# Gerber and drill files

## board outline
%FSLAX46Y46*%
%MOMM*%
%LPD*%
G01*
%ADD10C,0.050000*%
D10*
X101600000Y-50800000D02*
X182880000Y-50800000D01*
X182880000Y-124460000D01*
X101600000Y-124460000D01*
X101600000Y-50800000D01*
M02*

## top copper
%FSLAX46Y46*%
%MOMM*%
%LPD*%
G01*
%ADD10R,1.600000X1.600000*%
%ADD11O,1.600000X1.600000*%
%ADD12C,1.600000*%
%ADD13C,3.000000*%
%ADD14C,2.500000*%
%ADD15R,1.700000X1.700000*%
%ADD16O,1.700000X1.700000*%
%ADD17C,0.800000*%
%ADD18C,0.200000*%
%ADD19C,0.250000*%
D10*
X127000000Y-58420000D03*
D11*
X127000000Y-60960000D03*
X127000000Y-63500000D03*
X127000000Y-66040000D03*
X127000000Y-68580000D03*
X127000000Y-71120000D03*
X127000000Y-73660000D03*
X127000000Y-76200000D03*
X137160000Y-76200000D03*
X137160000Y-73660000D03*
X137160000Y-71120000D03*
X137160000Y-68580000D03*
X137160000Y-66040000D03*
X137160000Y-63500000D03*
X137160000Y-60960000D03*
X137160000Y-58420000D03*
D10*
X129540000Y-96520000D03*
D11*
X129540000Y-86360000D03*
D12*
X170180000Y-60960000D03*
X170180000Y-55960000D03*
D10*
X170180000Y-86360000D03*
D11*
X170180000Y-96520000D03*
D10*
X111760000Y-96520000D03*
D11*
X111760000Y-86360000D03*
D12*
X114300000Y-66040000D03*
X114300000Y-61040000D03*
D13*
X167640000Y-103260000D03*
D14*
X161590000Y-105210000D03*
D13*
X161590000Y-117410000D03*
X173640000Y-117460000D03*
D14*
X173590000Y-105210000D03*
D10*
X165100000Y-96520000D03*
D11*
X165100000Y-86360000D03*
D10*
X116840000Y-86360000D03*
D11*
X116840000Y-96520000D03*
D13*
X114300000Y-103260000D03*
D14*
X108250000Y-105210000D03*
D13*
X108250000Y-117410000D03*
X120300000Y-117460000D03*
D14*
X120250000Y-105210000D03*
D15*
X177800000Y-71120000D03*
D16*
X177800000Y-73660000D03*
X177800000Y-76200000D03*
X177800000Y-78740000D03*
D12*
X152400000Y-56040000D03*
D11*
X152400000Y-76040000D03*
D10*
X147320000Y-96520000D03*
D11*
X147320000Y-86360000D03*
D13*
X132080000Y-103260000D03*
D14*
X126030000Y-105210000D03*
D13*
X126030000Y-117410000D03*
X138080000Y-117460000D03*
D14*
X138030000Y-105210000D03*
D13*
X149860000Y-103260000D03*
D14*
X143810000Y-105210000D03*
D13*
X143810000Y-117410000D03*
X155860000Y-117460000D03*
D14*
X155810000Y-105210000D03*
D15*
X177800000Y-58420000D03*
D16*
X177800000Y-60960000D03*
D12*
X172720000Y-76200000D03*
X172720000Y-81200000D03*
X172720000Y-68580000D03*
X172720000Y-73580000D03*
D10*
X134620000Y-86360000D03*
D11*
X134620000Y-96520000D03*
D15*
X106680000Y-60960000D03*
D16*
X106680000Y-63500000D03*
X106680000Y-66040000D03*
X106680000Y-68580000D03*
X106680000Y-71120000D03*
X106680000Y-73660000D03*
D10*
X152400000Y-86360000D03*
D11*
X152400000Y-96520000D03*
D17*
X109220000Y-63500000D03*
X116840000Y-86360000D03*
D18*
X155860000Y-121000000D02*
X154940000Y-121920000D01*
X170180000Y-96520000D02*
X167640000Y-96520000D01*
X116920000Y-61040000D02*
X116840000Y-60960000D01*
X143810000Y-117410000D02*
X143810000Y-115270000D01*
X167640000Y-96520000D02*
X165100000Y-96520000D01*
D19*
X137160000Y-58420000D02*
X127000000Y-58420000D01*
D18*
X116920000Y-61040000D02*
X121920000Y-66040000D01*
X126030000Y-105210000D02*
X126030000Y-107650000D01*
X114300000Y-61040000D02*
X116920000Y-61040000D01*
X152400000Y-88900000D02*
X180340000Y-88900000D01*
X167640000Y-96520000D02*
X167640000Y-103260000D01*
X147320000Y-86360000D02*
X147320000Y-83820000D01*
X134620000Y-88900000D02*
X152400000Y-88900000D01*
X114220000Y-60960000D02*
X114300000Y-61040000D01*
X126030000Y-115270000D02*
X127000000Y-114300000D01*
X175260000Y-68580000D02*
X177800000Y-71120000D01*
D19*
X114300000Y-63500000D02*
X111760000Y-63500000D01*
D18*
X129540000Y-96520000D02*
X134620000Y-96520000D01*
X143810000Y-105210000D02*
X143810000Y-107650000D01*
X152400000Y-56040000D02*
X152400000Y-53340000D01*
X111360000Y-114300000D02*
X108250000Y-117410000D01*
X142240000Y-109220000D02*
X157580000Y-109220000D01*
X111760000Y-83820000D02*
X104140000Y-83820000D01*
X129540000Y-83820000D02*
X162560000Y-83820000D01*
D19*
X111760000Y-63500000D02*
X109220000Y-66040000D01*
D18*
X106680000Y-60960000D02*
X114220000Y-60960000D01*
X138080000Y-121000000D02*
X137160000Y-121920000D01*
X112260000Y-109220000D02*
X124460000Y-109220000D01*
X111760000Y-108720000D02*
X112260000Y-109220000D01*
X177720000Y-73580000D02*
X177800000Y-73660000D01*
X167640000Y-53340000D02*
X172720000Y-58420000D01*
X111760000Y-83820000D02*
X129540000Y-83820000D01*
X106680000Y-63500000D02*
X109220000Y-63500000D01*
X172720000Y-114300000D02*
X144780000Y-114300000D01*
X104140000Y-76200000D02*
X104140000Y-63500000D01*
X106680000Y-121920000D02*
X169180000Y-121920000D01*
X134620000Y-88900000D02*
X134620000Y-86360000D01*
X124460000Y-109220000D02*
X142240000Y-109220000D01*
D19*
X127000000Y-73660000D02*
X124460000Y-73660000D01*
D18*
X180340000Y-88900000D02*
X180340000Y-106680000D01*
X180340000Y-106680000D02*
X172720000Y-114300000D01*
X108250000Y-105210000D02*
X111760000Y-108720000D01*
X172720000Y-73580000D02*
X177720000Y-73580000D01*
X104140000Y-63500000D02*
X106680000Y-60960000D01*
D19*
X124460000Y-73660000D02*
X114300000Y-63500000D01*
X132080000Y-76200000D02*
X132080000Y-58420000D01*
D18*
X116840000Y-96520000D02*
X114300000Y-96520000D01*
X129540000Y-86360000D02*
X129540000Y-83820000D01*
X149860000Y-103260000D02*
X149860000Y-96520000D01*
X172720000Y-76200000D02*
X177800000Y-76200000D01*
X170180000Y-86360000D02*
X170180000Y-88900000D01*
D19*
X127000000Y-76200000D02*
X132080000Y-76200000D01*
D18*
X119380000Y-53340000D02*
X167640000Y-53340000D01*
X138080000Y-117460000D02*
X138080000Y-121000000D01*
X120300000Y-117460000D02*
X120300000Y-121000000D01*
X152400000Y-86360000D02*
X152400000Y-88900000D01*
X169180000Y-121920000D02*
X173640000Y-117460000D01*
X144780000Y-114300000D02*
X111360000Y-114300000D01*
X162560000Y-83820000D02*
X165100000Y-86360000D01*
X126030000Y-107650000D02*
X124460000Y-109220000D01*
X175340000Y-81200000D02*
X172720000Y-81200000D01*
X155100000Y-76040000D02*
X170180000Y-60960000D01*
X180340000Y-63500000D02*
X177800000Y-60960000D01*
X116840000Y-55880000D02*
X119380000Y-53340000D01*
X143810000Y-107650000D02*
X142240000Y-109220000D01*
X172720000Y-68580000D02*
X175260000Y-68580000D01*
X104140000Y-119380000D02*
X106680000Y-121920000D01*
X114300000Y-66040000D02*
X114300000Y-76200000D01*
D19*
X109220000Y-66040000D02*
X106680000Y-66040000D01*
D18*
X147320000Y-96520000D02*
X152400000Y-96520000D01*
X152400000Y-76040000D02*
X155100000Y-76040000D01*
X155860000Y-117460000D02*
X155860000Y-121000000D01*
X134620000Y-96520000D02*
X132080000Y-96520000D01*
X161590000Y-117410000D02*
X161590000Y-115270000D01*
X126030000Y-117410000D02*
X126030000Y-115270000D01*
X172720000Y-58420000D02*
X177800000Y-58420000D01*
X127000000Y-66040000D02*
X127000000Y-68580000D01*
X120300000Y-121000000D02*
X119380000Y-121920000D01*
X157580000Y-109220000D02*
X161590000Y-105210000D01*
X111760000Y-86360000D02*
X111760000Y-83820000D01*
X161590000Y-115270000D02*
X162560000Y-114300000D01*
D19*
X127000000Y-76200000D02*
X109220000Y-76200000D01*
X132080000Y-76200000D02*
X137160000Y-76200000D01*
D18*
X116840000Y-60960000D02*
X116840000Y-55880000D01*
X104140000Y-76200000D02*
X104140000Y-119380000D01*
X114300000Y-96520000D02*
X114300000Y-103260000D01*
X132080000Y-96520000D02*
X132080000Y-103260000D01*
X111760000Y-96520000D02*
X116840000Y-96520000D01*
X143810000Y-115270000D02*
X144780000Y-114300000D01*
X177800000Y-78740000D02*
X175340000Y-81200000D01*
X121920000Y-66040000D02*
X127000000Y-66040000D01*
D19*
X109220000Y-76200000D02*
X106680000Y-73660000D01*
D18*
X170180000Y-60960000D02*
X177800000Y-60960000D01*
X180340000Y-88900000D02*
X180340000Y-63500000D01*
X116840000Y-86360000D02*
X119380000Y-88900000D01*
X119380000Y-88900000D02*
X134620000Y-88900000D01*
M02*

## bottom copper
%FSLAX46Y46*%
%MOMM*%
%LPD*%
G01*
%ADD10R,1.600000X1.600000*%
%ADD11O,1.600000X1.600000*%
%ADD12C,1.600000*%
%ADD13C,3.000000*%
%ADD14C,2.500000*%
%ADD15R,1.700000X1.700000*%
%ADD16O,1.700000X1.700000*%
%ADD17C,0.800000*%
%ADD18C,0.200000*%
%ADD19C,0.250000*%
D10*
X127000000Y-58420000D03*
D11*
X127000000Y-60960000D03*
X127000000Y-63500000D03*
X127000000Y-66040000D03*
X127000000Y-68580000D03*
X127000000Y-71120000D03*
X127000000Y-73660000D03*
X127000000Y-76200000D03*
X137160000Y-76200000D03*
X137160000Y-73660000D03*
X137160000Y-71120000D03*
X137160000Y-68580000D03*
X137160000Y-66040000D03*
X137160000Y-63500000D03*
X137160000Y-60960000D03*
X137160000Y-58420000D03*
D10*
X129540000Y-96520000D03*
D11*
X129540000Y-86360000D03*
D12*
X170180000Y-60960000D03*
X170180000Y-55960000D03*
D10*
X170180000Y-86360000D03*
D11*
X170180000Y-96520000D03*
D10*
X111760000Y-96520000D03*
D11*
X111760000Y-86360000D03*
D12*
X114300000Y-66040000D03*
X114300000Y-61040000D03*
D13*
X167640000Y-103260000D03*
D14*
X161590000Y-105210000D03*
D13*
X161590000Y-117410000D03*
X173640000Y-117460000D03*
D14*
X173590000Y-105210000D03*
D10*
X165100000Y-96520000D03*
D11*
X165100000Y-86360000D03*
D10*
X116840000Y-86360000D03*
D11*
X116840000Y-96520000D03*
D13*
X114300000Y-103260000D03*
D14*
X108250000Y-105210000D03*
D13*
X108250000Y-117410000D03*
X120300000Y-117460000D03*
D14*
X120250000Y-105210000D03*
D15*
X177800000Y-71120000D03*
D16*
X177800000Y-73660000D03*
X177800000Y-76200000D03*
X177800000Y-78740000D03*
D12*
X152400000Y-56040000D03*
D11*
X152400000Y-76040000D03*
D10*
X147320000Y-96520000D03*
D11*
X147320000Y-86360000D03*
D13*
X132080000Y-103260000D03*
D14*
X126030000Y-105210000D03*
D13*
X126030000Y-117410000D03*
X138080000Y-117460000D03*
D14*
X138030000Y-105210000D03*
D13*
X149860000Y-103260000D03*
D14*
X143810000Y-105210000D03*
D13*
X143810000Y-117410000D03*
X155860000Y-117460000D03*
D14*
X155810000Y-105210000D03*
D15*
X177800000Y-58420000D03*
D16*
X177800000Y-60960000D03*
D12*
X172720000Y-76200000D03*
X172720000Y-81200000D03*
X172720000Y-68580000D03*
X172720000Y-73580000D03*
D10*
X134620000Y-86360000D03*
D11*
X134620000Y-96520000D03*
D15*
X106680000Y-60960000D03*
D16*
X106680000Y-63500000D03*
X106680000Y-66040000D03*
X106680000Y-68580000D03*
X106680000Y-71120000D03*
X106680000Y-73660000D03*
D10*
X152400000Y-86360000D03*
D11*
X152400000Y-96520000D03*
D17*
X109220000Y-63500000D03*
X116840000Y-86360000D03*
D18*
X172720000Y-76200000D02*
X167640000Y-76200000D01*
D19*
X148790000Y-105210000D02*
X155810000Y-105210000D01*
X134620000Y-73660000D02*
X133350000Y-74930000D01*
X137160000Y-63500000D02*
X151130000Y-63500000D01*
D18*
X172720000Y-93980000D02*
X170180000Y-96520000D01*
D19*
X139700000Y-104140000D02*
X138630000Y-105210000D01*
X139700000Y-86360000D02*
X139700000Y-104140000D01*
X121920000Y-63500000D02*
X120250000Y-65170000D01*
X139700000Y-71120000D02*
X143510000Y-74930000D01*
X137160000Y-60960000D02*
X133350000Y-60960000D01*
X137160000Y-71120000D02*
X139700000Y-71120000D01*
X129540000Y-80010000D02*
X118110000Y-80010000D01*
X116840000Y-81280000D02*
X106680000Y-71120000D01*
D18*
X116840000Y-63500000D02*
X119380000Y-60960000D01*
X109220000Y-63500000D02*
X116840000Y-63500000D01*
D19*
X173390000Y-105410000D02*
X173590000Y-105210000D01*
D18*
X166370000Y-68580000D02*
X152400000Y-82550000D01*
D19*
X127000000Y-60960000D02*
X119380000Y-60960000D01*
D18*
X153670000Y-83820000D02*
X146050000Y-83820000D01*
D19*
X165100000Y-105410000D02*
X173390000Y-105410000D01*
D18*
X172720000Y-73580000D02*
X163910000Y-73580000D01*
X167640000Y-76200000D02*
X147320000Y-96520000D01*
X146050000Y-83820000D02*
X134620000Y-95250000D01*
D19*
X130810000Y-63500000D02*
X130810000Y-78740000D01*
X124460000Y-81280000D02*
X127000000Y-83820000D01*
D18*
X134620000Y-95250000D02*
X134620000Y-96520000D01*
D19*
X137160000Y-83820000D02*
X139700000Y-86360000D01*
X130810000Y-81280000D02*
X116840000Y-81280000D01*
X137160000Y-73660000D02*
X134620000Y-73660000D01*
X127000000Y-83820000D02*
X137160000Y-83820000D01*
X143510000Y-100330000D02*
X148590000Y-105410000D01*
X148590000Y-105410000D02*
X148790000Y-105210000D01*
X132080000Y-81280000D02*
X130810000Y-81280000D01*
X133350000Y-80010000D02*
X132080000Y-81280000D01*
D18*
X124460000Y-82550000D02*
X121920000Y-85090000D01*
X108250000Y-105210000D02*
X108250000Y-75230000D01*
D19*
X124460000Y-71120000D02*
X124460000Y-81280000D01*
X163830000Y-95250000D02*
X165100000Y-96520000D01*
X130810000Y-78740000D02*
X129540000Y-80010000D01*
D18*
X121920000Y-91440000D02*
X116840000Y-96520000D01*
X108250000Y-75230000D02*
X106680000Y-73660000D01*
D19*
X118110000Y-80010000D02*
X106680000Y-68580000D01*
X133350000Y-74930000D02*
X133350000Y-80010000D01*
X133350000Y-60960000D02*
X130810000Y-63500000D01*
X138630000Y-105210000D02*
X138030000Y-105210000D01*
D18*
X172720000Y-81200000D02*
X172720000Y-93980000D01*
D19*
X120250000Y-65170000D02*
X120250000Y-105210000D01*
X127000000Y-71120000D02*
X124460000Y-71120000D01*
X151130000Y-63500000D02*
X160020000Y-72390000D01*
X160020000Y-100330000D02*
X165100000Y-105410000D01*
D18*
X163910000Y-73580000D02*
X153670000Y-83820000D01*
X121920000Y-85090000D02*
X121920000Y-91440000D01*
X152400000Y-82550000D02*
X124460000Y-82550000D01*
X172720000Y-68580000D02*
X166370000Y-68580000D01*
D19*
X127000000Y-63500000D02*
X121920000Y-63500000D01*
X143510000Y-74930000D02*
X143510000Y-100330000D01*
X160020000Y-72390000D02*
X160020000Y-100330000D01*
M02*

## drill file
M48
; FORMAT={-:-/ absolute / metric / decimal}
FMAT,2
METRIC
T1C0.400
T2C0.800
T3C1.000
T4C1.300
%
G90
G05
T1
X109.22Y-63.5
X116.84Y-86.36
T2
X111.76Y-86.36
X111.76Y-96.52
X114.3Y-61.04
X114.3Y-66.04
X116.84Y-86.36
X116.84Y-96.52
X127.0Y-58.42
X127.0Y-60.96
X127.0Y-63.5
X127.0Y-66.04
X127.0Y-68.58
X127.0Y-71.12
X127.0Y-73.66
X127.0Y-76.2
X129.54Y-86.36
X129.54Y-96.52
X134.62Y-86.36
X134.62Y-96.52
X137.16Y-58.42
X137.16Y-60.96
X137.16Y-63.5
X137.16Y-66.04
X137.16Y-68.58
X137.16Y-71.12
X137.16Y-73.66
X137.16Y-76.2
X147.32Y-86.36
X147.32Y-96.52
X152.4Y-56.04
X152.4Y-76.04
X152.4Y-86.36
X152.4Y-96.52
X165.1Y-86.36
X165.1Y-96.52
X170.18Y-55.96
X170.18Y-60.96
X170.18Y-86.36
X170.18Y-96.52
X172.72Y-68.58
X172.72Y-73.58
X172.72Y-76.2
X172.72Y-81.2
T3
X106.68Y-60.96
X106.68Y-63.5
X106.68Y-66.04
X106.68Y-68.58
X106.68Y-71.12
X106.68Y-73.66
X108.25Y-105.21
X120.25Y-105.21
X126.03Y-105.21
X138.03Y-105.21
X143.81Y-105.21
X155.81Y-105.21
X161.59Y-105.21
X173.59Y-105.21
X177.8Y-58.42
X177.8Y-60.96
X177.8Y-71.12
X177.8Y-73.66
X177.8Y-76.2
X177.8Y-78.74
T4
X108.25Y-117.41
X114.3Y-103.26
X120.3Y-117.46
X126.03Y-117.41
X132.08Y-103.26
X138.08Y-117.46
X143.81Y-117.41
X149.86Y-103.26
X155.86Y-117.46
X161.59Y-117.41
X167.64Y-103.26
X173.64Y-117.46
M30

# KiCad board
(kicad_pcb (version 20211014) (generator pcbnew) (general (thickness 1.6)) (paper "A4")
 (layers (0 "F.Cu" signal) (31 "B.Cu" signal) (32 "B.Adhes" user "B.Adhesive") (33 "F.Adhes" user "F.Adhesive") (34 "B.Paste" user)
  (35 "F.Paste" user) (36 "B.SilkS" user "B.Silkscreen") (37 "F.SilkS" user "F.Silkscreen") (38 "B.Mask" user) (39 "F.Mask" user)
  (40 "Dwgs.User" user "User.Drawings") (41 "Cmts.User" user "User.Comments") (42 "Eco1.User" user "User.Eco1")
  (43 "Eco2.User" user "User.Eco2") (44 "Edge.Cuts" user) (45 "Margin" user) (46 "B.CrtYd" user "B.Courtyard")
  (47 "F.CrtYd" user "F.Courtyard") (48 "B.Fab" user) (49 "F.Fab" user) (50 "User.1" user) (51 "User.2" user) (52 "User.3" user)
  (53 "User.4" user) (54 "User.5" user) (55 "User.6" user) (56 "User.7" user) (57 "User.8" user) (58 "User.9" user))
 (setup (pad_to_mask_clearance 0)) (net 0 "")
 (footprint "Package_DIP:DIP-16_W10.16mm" (layer "F.Cu") (at 127 58.42)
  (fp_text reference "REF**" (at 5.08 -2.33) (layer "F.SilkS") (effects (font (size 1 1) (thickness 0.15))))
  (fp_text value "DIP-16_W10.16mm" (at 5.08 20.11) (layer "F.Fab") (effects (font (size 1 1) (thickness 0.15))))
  (pad "1" thru_hole rect (at 0 0) (size 1.6 1.6) (drill 0.8) (layers *.Cu *.Mask))
  (pad "2" thru_hole oval (at 0 2.54) (size 1.6 1.6) (drill 0.8) (layers *.Cu *.Mask))
  (pad "3" thru_hole oval (at 0 5.08) (size 1.6 1.6) (drill 0.8) (layers *.Cu *.Mask))
  (pad "4" thru_hole oval (at 0 7.62) (size 1.6 1.6) (drill 0.8) (layers *.Cu *.Mask))
  (pad "5" thru_hole oval (at 0 10.16) (size 1.6 1.6) (drill 0.8) (layers *.Cu *.Mask))
  (pad "6" thru_hole oval (at 0 12.7) (size 1.6 1.6) (drill 0.8) (layers *.Cu *.Mask))
  (pad "7" thru_hole oval (at 0 15.24) (size 1.6 1.6) (drill 0.8) (layers *.Cu *.Mask))
  (pad "8" thru_hole oval (at 0 17.78) (size 1.6 1.6) (drill 0.8) (layers *.Cu *.Mask))
  (pad "9" thru_hole oval (at 10.16 17.78) (size 1.6 1.6) (drill 0.8) (layers *.Cu *.Mask))
  (pad "10" thru_hole oval (at 10.16 15.24) (size 1.6 1.6) (drill 0.8) (layers *.Cu *.Mask))
  (pad "11" thru_hole oval (at 10.16 12.7) (size 1.6 1.6) (drill 0.8) (layers *.Cu *.Mask))
  (pad "12" thru_hole oval (at 10.16 10.16) (size 1.6 1.6) (drill 0.8) (layers *.Cu *.Mask))
  (pad "13" thru_hole oval (at 10.16 7.62) (size 1.6 1.6) (drill 0.8) (layers *.Cu *.Mask))
  (pad "14" thru_hole oval (at 10.16 5.08) (size 1.6 1.6) (drill 0.8) (layers *.Cu *.Mask))
  (pad "15" thru_hole oval (at 10.16 2.54) (size 1.6 1.6) (drill 0.8) (layers *.Cu *.Mask))
  (pad "16" thru_hole oval (at 10.16 0) (size 1.6 1.6) (drill 0.8) (layers *.Cu *.Mask)))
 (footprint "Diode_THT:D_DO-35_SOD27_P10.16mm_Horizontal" (layer "F.Cu") (at 129.54 96.52 90)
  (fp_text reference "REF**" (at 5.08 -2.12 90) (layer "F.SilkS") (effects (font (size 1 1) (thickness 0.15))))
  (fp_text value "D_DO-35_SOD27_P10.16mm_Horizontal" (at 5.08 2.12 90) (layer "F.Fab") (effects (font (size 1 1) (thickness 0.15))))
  (pad "1" thru_hole rect (at 0 0 90) (size 1.6 1.6) (drill 0.8) (layers *.Cu *.Mask))
  (pad "2" thru_hole oval (at 10.16 0 90) (size 1.6 1.6) (drill 0.8) (layers *.Cu *.Mask)))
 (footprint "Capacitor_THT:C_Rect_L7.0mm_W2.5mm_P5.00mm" (layer "F.Cu") (at 170.18 60.96 90)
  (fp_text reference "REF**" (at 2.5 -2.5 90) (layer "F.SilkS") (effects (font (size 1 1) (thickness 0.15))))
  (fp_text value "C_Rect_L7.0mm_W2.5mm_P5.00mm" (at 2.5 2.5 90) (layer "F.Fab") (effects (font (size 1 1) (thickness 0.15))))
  (pad "1" thru_hole circle (at 0 0 90) (size 1.6 1.6) (drill 0.8) (layers *.Cu *.Mask))
  (pad "2" thru_hole circle (at 5 0 90) (size 1.6 1.6) (drill 0.8) (layers *.Cu *.Mask)))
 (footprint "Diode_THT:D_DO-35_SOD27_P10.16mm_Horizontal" (layer "F.Cu") (at 170.18 86.36 -90)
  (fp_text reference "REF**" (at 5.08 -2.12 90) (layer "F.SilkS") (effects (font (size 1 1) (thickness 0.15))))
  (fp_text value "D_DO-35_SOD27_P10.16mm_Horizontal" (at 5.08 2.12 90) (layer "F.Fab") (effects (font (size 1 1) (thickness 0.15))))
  (pad "1" thru_hole rect (at 0 0 270) (size 1.6 1.6) (drill 0.8) (layers *.Cu *.Mask))
  (pad "2" thru_hole oval (at 10.16 0 270) (size 1.6 1.6) (drill 0.8) (layers *.Cu *.Mask)))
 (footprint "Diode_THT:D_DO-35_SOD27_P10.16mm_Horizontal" (layer "F.Cu") (at 111.76 96.52 90)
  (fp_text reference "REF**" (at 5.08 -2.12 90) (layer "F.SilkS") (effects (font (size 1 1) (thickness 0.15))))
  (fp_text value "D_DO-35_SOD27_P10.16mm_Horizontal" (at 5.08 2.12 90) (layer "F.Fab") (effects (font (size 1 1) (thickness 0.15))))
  (pad "1" thru_hole rect (at 0 0 90) (size 1.6 1.6) (drill 0.8) (layers *.Cu *.Mask))
  (pad "2" thru_hole oval (at 10.16 0 90) (size 1.6 1.6) (drill 0.8) (layers *.Cu *.Mask)))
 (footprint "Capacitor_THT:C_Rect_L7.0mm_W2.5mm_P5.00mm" (layer "F.Cu") (at 114.3 66.04 90)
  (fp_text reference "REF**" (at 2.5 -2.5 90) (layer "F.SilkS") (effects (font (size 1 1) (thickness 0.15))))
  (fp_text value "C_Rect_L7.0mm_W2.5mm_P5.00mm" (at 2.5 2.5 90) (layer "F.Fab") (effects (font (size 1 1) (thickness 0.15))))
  (pad "1" thru_hole circle (at 0 0 90) (size 1.6 1.6) (drill 0.8) (layers *.Cu *.Mask))
  (pad "2" thru_hole circle (at 5 0 90) (size 1.6 1.6) (drill 0.8) (layers *.Cu *.Mask)))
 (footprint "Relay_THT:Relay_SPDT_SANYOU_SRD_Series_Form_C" (layer "F.Cu") (at 167.64 103.26 -90)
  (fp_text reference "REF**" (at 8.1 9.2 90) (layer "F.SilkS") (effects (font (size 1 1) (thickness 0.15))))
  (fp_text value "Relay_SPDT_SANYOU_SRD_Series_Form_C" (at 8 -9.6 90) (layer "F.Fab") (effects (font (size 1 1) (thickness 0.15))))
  (pad "1" thru_hole circle (at 0 0) (size 3 3) (drill 1.3) (layers *.Cu *.Mask))
  (pad "2" thru_hole circle (at 1.95 6.05) (size 2.5 2.5) (drill 1) (layers *.Cu *.Mask))
  (pad "3" thru_hole circle (at 14.15 6.05) (size 3 3) (drill 1.3) (layers *.Cu *.Mask))
  (pad "4" thru_hole circle (at 14.2 -6) (size 3 3) (drill 1.3) (layers *.Cu *.Mask))
  (pad "5" thru_hole circle (at 1.95 -5.95) (size 2.5 2.5) (drill 1) (layers *.Cu *.Mask)))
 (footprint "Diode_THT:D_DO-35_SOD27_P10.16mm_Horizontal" (layer "F.Cu") (at 165.1 96.52 90)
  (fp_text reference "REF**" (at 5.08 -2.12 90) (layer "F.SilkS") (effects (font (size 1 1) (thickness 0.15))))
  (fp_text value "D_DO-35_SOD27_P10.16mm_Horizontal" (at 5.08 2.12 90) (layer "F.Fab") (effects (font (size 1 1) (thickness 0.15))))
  (pad "1" thru_hole rect (at 0 0 90) (size 1.6 1.6) (drill 0.8) (layers *.Cu *.Mask))
  (pad "2" thru_hole oval (at 10.16 0 90) (size 1.6 1.6) (drill 0.8) (layers *.Cu *.Mask)))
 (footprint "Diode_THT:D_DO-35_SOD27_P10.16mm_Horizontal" (layer "F.Cu") (at 116.84 86.36 -90)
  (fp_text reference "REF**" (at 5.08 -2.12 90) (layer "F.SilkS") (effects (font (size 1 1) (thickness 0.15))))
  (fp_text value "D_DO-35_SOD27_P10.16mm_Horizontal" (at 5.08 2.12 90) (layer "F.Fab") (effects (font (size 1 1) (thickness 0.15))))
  (pad "1" thru_hole rect (at 0 0 270) (size 1.6 1.6) (drill 0.8) (layers *.Cu *.Mask))
  (pad "2" thru_hole oval (at 10.16 0 270) (size 1.6 1.6) (drill 0.8) (layers *.Cu *.Mask)))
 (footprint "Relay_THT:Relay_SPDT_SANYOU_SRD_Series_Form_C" (layer "F.Cu") (at 114.3 103.26 -90)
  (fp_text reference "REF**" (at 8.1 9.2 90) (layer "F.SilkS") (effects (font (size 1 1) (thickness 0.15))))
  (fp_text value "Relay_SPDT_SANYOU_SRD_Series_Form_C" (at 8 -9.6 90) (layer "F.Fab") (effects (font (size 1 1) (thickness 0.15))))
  (pad "1" thru_hole circle (at 0 0) (size 3 3) (drill 1.3) (layers *.Cu *.Mask))
  (pad "2" thru_hole circle (at 1.95 6.05) (size 2.5 2.5) (drill 1) (layers *.Cu *.Mask))
  (pad "3" thru_hole circle (at 14.15 6.05) (size 3 3) (drill 1.3) (layers *.Cu *.Mask))
  (pad "4" thru_hole circle (at 14.2 -6) (size 3 3) (drill 1.3) (layers *.Cu *.Mask))
  (pad "5" thru_hole circle (at 1.95 -5.95) (size 2.5 2.5) (drill 1) (layers *.Cu *.Mask)))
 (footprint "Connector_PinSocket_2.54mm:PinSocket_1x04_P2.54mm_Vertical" (layer "F.Cu") (at 177.8 71.12)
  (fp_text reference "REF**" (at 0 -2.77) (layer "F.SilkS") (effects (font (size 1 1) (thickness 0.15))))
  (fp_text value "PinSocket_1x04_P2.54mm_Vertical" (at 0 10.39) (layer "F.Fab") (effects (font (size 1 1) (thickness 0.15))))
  (pad "1" thru_hole rect (at 0 0) (size 1.7 1.7) (drill 1) (layers *.Cu *.Mask))
  (pad "2" thru_hole oval (at 0 2.54) (size 1.7 1.7) (drill 1) (layers *.Cu *.Mask))
  (pad "3" thru_hole oval (at 0 5.08) (size 1.7 1.7) (drill 1) (layers *.Cu *.Mask))
  (pad "4" thru_hole oval (at 0 7.62) (size 1.7 1.7) (drill 1) (layers *.Cu *.Mask)))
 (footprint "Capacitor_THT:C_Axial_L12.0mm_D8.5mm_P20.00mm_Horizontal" (layer "F.Cu") (at 152.4 56.04 -90)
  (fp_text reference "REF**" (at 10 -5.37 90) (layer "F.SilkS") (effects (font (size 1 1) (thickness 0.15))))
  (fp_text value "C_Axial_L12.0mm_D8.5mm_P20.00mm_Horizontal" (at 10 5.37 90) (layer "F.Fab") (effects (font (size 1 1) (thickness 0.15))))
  (pad "1" thru_hole circle (at 0 0 270) (size 1.6 1.6) (drill 0.8) (layers *.Cu *.Mask))
  (pad "2" thru_hole oval (at 20 0 270) (size 1.6 1.6) (drill 0.8) (layers *.Cu *.Mask)))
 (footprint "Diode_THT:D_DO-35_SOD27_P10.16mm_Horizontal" (layer "F.Cu") (at 147.32 96.52 90)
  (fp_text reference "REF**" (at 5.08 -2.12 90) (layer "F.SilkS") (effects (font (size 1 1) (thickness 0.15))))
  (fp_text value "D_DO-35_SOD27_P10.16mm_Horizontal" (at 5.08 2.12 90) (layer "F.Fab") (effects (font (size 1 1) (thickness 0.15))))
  (pad "1" thru_hole rect (at 0 0 90) (size 1.6 1.6) (drill 0.8) (layers *.Cu *.Mask))
  (pad "2" thru_hole oval (at 10.16 0 90) (size 1.6 1.6) (drill 0.8) (layers *.Cu *.Mask)))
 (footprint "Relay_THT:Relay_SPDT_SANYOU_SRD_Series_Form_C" (layer "F.Cu") (at 132.08 103.26 -90)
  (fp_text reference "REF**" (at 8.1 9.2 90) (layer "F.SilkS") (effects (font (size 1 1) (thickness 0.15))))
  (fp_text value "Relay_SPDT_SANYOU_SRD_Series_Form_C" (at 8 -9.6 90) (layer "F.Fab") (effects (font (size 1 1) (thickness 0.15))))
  (pad "1" thru_hole circle (at 0 0) (size 3 3) (drill 1.3) (layers *.Cu *.Mask))
  (pad "2" thru_hole circle (at 1.95 6.05) (size 2.5 2.5) (drill 1) (layers *.Cu *.Mask))
  (pad "3" thru_hole circle (at 14.15 6.05) (size 3 3) (drill 1.3) (layers *.Cu *.Mask))
  (pad "4" thru_hole circle (at 14.2 -6) (size 3 3) (drill 1.3) (layers *.Cu *.Mask))
  (pad "5" thru_hole circle (at 1.95 -5.95) (size 2.5 2.5) (drill 1) (layers *.Cu *.Mask)))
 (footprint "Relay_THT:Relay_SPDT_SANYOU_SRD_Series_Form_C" (layer "F.Cu") (at 149.86 103.26 -90)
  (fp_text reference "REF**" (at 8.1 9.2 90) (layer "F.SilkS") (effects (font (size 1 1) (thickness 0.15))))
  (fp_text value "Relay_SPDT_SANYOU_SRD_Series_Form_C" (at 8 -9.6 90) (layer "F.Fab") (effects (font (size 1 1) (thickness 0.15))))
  (pad "1" thru_hole circle (at 0 0) (size 3 3) (drill 1.3) (layers *.Cu *.Mask))
  (pad "2" thru_hole circle (at 1.95 6.05) (size 2.5 2.5) (drill 1) (layers *.Cu *.Mask))
  (pad "3" thru_hole circle (at 14.15 6.05) (size 3 3) (drill 1.3) (layers *.Cu *.Mask))
  (pad "4" thru_hole circle (at 14.2 -6) (size 3 3) (drill 1.3) (layers *.Cu *.Mask))
  (pad "5" thru_hole circle (at 1.95 -5.95) (size 2.5 2.5) (drill 1) (layers *.Cu *.Mask)))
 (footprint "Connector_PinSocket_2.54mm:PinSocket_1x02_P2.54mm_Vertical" (layer "F.Cu") (at 177.8 58.42)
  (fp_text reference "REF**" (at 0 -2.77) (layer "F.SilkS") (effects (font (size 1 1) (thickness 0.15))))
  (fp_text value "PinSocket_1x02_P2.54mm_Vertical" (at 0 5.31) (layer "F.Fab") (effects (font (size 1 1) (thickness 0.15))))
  (pad "1" thru_hole rect (at 0 0) (size 1.7 1.7) (drill 1) (layers *.Cu *.Mask))
  (pad "2" thru_hole oval (at 0 2.54) (size 1.7 1.7) (drill 1) (layers *.Cu *.Mask)))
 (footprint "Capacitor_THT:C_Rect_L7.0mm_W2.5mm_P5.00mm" (layer "F.Cu") (at 172.72 76.2 -90)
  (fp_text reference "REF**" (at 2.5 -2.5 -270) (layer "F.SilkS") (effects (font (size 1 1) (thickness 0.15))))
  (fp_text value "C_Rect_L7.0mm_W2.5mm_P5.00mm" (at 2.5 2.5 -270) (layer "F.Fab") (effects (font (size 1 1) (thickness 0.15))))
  (pad "1" thru_hole circle (at 0 0 270) (size 1.6 1.6) (drill 0.8) (layers *.Cu *.Mask))
  (pad "2" thru_hole circle (at 5 0 270) (size 1.6 1.6) (drill 0.8) (layers *.Cu *.Mask)))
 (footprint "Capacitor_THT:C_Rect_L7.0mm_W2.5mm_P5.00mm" (layer "F.Cu") (at 172.72 68.58 -90)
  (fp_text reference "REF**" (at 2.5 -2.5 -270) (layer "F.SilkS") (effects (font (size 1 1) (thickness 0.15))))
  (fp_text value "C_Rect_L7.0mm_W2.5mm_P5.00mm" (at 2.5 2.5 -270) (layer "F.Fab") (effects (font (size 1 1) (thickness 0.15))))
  (pad "1" thru_hole circle (at 0 0 270) (size 1.6 1.6) (drill 0.8) (layers *.Cu *.Mask))
  (pad "2" thru_hole circle (at 5 0 270) (size 1.6 1.6) (drill 0.8) (layers *.Cu *.Mask)))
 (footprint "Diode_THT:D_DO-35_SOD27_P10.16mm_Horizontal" (layer "F.Cu") (at 134.62 86.36 -90)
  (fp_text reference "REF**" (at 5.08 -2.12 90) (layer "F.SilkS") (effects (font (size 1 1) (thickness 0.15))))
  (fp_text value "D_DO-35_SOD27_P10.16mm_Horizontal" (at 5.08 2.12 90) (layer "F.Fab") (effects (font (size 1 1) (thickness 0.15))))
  (pad "1" thru_hole rect (at 0 0 270) (size 1.6 1.6) (drill 0.8) (layers *.Cu *.Mask))
  (pad "2" thru_hole oval (at 10.16 0 270) (size 1.6 1.6) (drill 0.8) (layers *.Cu *.Mask)))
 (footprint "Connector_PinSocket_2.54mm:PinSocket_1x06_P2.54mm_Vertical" (layer "F.Cu") (at 106.68 60.96)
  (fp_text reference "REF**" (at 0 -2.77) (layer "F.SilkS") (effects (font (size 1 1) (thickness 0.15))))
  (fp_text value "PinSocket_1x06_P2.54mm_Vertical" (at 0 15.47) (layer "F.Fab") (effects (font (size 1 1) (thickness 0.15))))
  (pad "1" thru_hole rect (at 0 0) (size 1.7 1.7) (drill 1) (layers *.Cu *.Mask))
  (pad "2" thru_hole oval (at 0 2.54) (size 1.7 1.7) (drill 1) (layers *.Cu *.Mask))
  (pad "3" thru_hole oval (at 0 5.08) (size 1.7 1.7) (drill 1) (layers *.Cu *.Mask))
  (pad "4" thru_hole oval (at 0 7.62) (size 1.7 1.7) (drill 1) (layers *.Cu *.Mask))
  (pad "5" thru_hole oval (at 0 10.16) (size 1.7 1.7) (drill 1) (layers *.Cu *.Mask))
  (pad "6" thru_hole oval (at 0 12.7) (size 1.7 1.7) (drill 1) (layers *.Cu *.Mask)))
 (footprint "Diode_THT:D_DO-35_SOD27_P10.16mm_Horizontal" (layer "F.Cu") (at 152.4 86.36 -90)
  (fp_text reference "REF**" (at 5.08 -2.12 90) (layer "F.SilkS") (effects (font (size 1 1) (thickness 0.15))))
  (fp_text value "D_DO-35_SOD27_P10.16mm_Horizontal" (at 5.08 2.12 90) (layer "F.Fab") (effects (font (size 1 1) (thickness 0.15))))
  (pad "1" thru_hole rect (at 0 0 270) (size 1.6 1.6) (drill 0.8) (layers *.Cu *.Mask))
  (pad "2" thru_hole oval (at 10.16 0 270) (size 1.6 1.6) (drill 0.8) (layers *.Cu *.Mask)))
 (gr_rect (start 101.6 50.8) (end 182.88 124.46) (layer "Edge.Cuts") (width 0.05) (fill none))
 (segment (start 155.86 121) (end 154.94 121.92) (width 0.2) (layer "F.Cu") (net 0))
 (segment (start 170.18 96.52) (end 167.64 96.52) (width 0.2) (layer "F.Cu") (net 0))
 (segment (start 116.92 61.04) (end 116.84 60.96) (width 0.2) (layer "F.Cu") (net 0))
 (segment (start 143.81 117.41) (end 143.81 115.27) (width 0.2) (layer "F.Cu") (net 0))
 (segment (start 167.64 96.52) (end 165.1 96.52) (width 0.2) (layer "F.Cu") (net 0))
 (segment (start 137.16 58.42) (end 127 58.42) (width 0.25) (layer "F.Cu") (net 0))
 (segment (start 116.92 61.04) (end 121.92 66.04) (width 0.2) (layer "F.Cu") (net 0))
 (segment (start 126.03 105.21) (end 126.03 107.65) (width 0.2) (layer "F.Cu") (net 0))
 (segment (start 114.3 61.04) (end 116.92 61.04) (width 0.2) (layer "F.Cu") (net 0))
 (segment (start 152.4 88.9) (end 180.34 88.9) (width 0.2) (layer "F.Cu") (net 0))
 (segment (start 167.64 96.52) (end 167.64 103.26) (width 0.2) (layer "F.Cu") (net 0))
 (segment (start 147.32 86.36) (end 147.32 83.82) (width 0.2) (layer "F.Cu") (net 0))
 (segment (start 134.62 88.9) (end 152.4 88.9) (width 0.2) (layer "F.Cu") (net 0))
 (segment (start 114.22 60.96) (end 114.3 61.04) (width 0.2) (layer "F.Cu") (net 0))
 (segment (start 126.03 115.27) (end 127 114.3) (width 0.2) (layer "F.Cu") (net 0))
 (segment (start 175.26 68.58) (end 177.8 71.12) (width 0.2) (layer "F.Cu") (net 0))
 (segment (start 114.3 63.5) (end 111.76 63.5) (width 0.25) (layer "F.Cu") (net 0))
 (segment (start 129.54 96.52) (end 134.62 96.52) (width 0.2) (layer "F.Cu") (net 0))
 (segment (start 143.81 105.21) (end 143.81 107.65) (width 0.2) (layer "F.Cu") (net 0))
 (segment (start 152.4 56.04) (end 152.4 53.34) (width 0.2) (layer "F.Cu") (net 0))
 (segment (start 111.36 114.3) (end 108.25 117.41) (width 0.2) (layer "F.Cu") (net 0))
 (segment (start 142.24 109.22) (end 157.58 109.22) (width 0.2) (layer "F.Cu") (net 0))
 (segment (start 111.76 83.82) (end 104.14 83.82) (width 0.2) (layer "F.Cu") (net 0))
 (segment (start 129.54 83.82) (end 162.56 83.82) (width 0.2) (layer "F.Cu") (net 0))
 (segment (start 111.76 63.5) (end 109.22 66.04) (width 0.25) (layer "F.Cu") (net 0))
 (segment (start 106.68 60.96) (end 114.22 60.96) (width 0.2) (layer "F.Cu") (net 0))
 (segment (start 138.08 121) (end 137.16 121.92) (width 0.2) (layer "F.Cu") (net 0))
 (segment (start 112.26 109.22) (end 124.46 109.22) (width 0.2) (layer "F.Cu") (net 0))
 (segment (start 111.76 108.72) (end 112.26 109.22) (width 0.2) (layer "F.Cu") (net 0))
 (segment (start 177.72 73.58) (end 177.8 73.66) (width 0.2) (layer "F.Cu") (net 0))
 (segment (start 167.64 53.34) (end 172.72 58.42) (width 0.2) (layer "F.Cu") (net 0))
 (segment (start 111.76 83.82) (end 129.54 83.82) (width 0.2) (layer "F.Cu") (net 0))
 (segment (start 106.68 63.5) (end 109.22 63.5) (width 0.2) (layer "F.Cu") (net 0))
 (segment (start 172.72 114.3) (end 144.78 114.3) (width 0.2) (layer "F.Cu") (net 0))
 (segment (start 104.14 76.2) (end 104.14 63.5) (width 0.2) (layer "F.Cu") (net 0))
 (segment (start 106.68 121.92) (end 169.18 121.92) (width 0.2) (layer "F.Cu") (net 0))
 (segment (start 134.62 88.9) (end 134.62 86.36) (width 0.2) (layer "F.Cu") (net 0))
 (segment (start 124.46 109.22) (end 142.24 109.22) (width 0.2) (layer "F.Cu") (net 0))
 (segment (start 127 73.66) (end 124.46 73.66) (width 0.25) (layer "F.Cu") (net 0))
 (segment (start 180.34 88.9) (end 180.34 106.68) (width 0.2) (layer "F.Cu") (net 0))
 (segment (start 180.34 106.68) (end 172.72 114.3) (width 0.2) (layer "F.Cu") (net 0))
 (segment (start 108.25 105.21) (end 111.76 108.72) (width 0.2) (layer "F.Cu") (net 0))
 (segment (start 172.72 73.58) (end 177.72 73.58) (width 0.2) (layer "F.Cu") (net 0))
 (segment (start 104.14 63.5) (end 106.68 60.96) (width 0.2) (layer "F.Cu") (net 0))
 (segment (start 124.46 73.66) (end 114.3 63.5) (width 0.25) (layer "F.Cu") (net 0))
 (segment (start 132.08 76.2) (end 132.08 58.42) (width 0.25) (layer "F.Cu") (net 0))
 (segment (start 116.84 96.52) (end 114.3 96.52) (width 0.2) (layer "F.Cu") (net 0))
 (segment (start 129.54 86.36) (end 129.54 83.82) (width 0.2) (layer "F.Cu") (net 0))
 (segment (start 149.86 103.26) (end 149.86 96.52) (width 0.2) (layer "F.Cu") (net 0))
 (segment (start 172.72 76.2) (end 177.8 76.2) (width 0.2) (layer "F.Cu") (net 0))
 (segment (start 170.18 86.36) (end 170.18 88.9) (width 0.2) (layer "F.Cu") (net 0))
 (segment (start 127 76.2) (end 132.08 76.2) (width 0.25) (layer "F.Cu") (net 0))
 (segment (start 119.38 53.34) (end 167.64 53.34) (width 0.2) (layer "F.Cu") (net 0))
 (segment (start 138.08 117.46) (end 138.08 121) (width 0.2) (layer "F.Cu") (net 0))
 (segment (start 120.3 117.46) (end 120.3 121) (width 0.2) (layer "F.Cu") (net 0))
 (segment (start 152.4 86.36) (end 152.4 88.9) (width 0.2) (layer "F.Cu") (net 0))
 (segment (start 169.18 121.92) (end 173.64 117.46) (width 0.2) (layer "F.Cu") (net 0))
 (segment (start 144.78 114.3) (end 111.36 114.3) (width 0.2) (layer "F.Cu") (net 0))
 (segment (start 162.56 83.82) (end 165.1 86.36) (width 0.2) (layer "F.Cu") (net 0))
 (segment (start 126.03 107.65) (end 124.46 109.22) (width 0.2) (layer "F.Cu") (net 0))
 (segment (start 175.34 81.2) (end 172.72 81.2) (width 0.2) (layer "F.Cu") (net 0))
 (segment (start 155.1 76.04) (end 170.18 60.96) (width 0.2) (layer "F.Cu") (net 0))
 (segment (start 180.34 63.5) (end 177.8 60.96) (width 0.2) (layer "F.Cu") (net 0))
 (segment (start 116.84 55.88) (end 119.38 53.34) (width 0.2) (layer "F.Cu") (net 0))
 (segment (start 143.81 107.65) (end 142.24 109.22) (width 0.2) (layer "F.Cu") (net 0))
 (segment (start 172.72 68.58) (end 175.26 68.58) (width 0.2) (layer "F.Cu") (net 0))
 (segment (start 104.14 119.38) (end 106.68 121.92) (width 0.2) (layer "F.Cu") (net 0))
 (segment (start 114.3 66.04) (end 114.3 76.2) (width 0.2) (layer "F.Cu") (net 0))
 (segment (start 109.22 66.04) (end 106.68 66.04) (width 0.25) (layer "F.Cu") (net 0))
 (segment (start 147.32 96.52) (end 152.4 96.52) (width 0.2) (layer "F.Cu") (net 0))
 (segment (start 152.4 76.04) (end 155.1 76.04) (width 0.2) (layer "F.Cu") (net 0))
 (segment (start 155.86 117.46) (end 155.86 121) (width 0.2) (layer "F.Cu") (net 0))
 (segment (start 134.62 96.52) (end 132.08 96.52) (width 0.2) (layer "F.Cu") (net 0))
 (segment (start 161.59 117.41) (end 161.59 115.27) (width 0.2) (layer "F.Cu") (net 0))
 (segment (start 126.03 117.41) (end 126.03 115.27) (width 0.2) (layer "F.Cu") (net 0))
 (segment (start 172.72 58.42) (end 177.8 58.42) (width 0.2) (layer "F.Cu") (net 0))
 (segment (start 127 66.04) (end 127 68.58) (width 0.2) (layer "F.Cu") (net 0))
 (segment (start 120.3 121) (end 119.38 121.92) (width 0.2) (layer "F.Cu") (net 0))
 (segment (start 157.58 109.22) (end 161.59 105.21) (width 0.2) (layer "F.Cu") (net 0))
 (segment (start 111.76 86.36) (end 111.76 83.82) (width 0.2) (layer "F.Cu") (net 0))
 (segment (start 161.59 115.27) (end 162.56 114.3) (width 0.2) (layer "F.Cu") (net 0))
 (segment (start 127 76.2) (end 109.22 76.2) (width 0.25) (layer "F.Cu") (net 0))
 (segment (start 132.08 76.2) (end 137.16 76.2) (width 0.25) (layer "F.Cu") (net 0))
 (segment (start 116.84 60.96) (end 116.84 55.88) (width 0.2) (layer "F.Cu") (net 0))
 (segment (start 104.14 76.2) (end 104.14 119.38) (width 0.2) (layer "F.Cu") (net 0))
 (segment (start 114.3 96.52) (end 114.3 103.26) (width 0.2) (layer "F.Cu") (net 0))
 (segment (start 132.08 96.52) (end 132.08 103.26) (width 0.2) (layer "F.Cu") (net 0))
 (segment (start 111.76 96.52) (end 116.84 96.52) (width 0.2) (layer "F.Cu") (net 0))
 (segment (start 143.81 115.27) (end 144.78 114.3) (width 0.2) (layer "F.Cu") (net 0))
 (segment (start 177.8 78.74) (end 175.34 81.2) (width 0.2) (layer "F.Cu") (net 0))
 (segment (start 121.92 66.04) (end 127 66.04) (width 0.2) (layer "F.Cu") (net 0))
 (segment (start 109.22 76.2) (end 106.68 73.66) (width 0.25) (layer "F.Cu") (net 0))
 (segment (start 170.18 60.96) (end 177.8 60.96) (width 0.2) (layer "F.Cu") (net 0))
 (segment (start 180.34 88.9) (end 180.34 63.5) (width 0.2) (layer "F.Cu") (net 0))
 (segment (start 116.84 86.36) (end 119.38 88.9) (width 0.2) (layer "F.Cu") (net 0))
 (segment (start 119.38 88.9) (end 134.62 88.9) (width 0.2) (layer "F.Cu") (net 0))
 (via (at 109.22 63.5) (size 0.8) (drill 0.4) (layers "F.Cu" "B.Cu") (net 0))
 (via (at 116.84 86.36) (size 0.8) (drill 0.4) (layers "F.Cu" "B.Cu") (free) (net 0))
 (segment (start 172.72 76.2) (end 167.64 76.2) (width 0.2) (layer "B.Cu") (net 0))
 (segment (start 148.79 105.21) (end 155.81 105.21) (width 0.25) (layer "B.Cu") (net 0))
 (segment (start 134.62 73.66) (end 133.35 74.93) (width 0.25) (layer "B.Cu") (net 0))
 (segment (start 137.16 63.5) (end 151.13 63.5) (width 0.25) (layer "B.Cu") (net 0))
 (segment (start 172.72 93.98) (end 170.18 96.52) (width 0.2) (layer "B.Cu") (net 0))
 (segment (start 139.7 104.14) (end 138.63 105.21) (width 0.25) (layer "B.Cu") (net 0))
 (segment (start 139.7 86.36) (end 139.7 104.14) (width 0.25) (layer "B.Cu") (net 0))
 (segment (start 121.92 63.5) (end 120.25 65.17) (width 0.25) (layer "B.Cu") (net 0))
 (segment (start 139.7 71.12) (end 143.51 74.93) (width 0.25) (layer "B.Cu") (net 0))
 (segment (start 137.16 60.96) (end 133.35 60.96) (width 0.25) (layer "B.Cu") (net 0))
 (segment (start 137.16 71.12) (end 139.7 71.12) (width 0.25) (layer "B.Cu") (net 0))
 (segment (start 129.54 80.01) (end 118.11 80.01) (width 0.25) (layer "B.Cu") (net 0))
 (segment (start 116.84 81.28) (end 106.68 71.12) (width 0.25) (layer "B.Cu") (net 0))
 (segment (start 116.84 63.5) (end 119.38 60.96) (width 0.2) (layer "B.Cu") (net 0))
 (segment (start 109.22 63.5) (end 116.84 63.5) (width 0.2) (layer "B.Cu") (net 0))
 (segment (start 173.39 105.41) (end 173.59 105.21) (width 0.25) (layer "B.Cu") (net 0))
 (segment (start 166.37 68.58) (end 152.4 82.55) (width 0.2) (layer "B.Cu") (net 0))
 (segment (start 127 60.96) (end 119.38 60.96) (width 0.25) (layer "B.Cu") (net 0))
 (segment (start 153.67 83.82) (end 146.05 83.82) (width 0.2) (layer "B.Cu") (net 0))
 (segment (start 165.1 105.41) (end 173.39 105.41) (width 0.25) (layer "B.Cu") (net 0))
 (segment (start 172.72 73.58) (end 163.91 73.58) (width 0.2) (layer "B.Cu") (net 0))
 (segment (start 167.64 76.2) (end 147.32 96.52) (width 0.2) (layer "B.Cu") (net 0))
 (segment (start 146.05 83.82) (end 134.62 95.25) (width 0.2) (layer "B.Cu") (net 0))
 (segment (start 130.81 63.5) (end 130.81 78.74) (width 0.25) (layer "B.Cu") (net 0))
 (segment (start 124.46 81.28) (end 127 83.82) (width 0.25) (layer "B.Cu") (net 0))
 (segment (start 134.62 95.25) (end 134.62 96.52) (width 0.2) (layer "B.Cu") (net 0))
 (segment (start 137.16 83.82) (end 139.7 86.36) (width 0.25) (layer "B.Cu") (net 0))
 (segment (start 130.81 81.28) (end 116.84 81.28) (width 0.25) (layer "B.Cu") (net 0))
 (segment (start 137.16 73.66) (end 134.62 73.66) (width 0.25) (layer "B.Cu") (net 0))
 (segment (start 127 83.82) (end 137.16 83.82) (width 0.25) (layer "B.Cu") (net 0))
 (segment (start 143.51 100.33) (end 148.59 105.41) (width 0.25) (layer "B.Cu") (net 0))
 (segment (start 148.59 105.41) (end 148.79 105.21) (width 0.25) (layer "B.Cu") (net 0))
 (segment (start 132.08 81.28) (end 130.81 81.28) (width 0.25) (layer "B.Cu") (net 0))
 (segment (start 133.35 80.01) (end 132.08 81.28) (width 0.25) (layer "B.Cu") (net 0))
 (segment (start 124.46 82.55) (end 121.92 85.09) (width 0.2) (layer "B.Cu") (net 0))
 (segment (start 108.25 105.21) (end 108.25 75.23) (width 0.2) (layer "B.Cu") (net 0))
 (segment (start 124.46 71.12) (end 124.46 81.28) (width 0.25) (layer "B.Cu") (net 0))
 (segment (start 163.83 95.25) (end 165.1 96.52) (width 0.25) (layer "B.Cu") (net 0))
 (segment (start 130.81 78.74) (end 129.54 80.01) (width 0.25) (layer "B.Cu") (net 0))
 (segment (start 121.92 91.44) (end 116.84 96.52) (width 0.2) (layer "B.Cu") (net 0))
 (segment (start 108.25 75.23) (end 106.68 73.66) (width 0.2) (layer "B.Cu") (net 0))
 (segment (start 118.11 80.01) (end 106.68 68.58) (width 0.25) (layer "B.Cu") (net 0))
 (segment (start 133.35 74.93) (end 133.35 80.01) (width 0.25) (layer "B.Cu") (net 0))
 (segment (start 133.35 60.96) (end 130.81 63.5) (width 0.25) (layer "B.Cu") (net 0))
 (segment (start 138.63 105.21) (end 138.03 105.21) (width 0.25) (layer "B.Cu") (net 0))
 (segment (start 172.72 81.2) (end 172.72 93.98) (width 0.2) (layer "B.Cu") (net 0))
 (segment (start 120.25 65.17) (end 120.25 105.21) (width 0.25) (layer "B.Cu") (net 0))
 (segment (start 127 71.12) (end 124.46 71.12) (width 0.25) (layer "B.Cu") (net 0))
 (segment (start 151.13 63.5) (end 160.02 72.39) (width 0.25) (layer "B.Cu") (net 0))
 (segment (start 160.02 100.33) (end 165.1 105.41) (width 0.25) (layer "B.Cu") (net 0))
 (segment (start 163.91 73.58) (end 153.67 83.82) (width 0.2) (layer "B.Cu") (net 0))
 (segment (start 121.92 85.09) (end 121.92 91.44) (width 0.2) (layer "B.Cu") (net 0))
 (segment (start 152.4 82.55) (end 124.46 82.55) (width 0.2) (layer "B.Cu") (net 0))
 (segment (start 172.72 68.58) (end 166.37 68.58) (width 0.2) (layer "B.Cu") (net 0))
 (segment (start 127 63.5) (end 121.92 63.5) (width 0.25) (layer "B.Cu") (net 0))
 (segment (start 143.51 74.93) (end 143.51 100.33) (width 0.25) (layer "B.Cu") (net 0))
 (segment (start 160.02 72.39) (end 160.02 100.33) (width 0.25) (layer "B.Cu") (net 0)))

